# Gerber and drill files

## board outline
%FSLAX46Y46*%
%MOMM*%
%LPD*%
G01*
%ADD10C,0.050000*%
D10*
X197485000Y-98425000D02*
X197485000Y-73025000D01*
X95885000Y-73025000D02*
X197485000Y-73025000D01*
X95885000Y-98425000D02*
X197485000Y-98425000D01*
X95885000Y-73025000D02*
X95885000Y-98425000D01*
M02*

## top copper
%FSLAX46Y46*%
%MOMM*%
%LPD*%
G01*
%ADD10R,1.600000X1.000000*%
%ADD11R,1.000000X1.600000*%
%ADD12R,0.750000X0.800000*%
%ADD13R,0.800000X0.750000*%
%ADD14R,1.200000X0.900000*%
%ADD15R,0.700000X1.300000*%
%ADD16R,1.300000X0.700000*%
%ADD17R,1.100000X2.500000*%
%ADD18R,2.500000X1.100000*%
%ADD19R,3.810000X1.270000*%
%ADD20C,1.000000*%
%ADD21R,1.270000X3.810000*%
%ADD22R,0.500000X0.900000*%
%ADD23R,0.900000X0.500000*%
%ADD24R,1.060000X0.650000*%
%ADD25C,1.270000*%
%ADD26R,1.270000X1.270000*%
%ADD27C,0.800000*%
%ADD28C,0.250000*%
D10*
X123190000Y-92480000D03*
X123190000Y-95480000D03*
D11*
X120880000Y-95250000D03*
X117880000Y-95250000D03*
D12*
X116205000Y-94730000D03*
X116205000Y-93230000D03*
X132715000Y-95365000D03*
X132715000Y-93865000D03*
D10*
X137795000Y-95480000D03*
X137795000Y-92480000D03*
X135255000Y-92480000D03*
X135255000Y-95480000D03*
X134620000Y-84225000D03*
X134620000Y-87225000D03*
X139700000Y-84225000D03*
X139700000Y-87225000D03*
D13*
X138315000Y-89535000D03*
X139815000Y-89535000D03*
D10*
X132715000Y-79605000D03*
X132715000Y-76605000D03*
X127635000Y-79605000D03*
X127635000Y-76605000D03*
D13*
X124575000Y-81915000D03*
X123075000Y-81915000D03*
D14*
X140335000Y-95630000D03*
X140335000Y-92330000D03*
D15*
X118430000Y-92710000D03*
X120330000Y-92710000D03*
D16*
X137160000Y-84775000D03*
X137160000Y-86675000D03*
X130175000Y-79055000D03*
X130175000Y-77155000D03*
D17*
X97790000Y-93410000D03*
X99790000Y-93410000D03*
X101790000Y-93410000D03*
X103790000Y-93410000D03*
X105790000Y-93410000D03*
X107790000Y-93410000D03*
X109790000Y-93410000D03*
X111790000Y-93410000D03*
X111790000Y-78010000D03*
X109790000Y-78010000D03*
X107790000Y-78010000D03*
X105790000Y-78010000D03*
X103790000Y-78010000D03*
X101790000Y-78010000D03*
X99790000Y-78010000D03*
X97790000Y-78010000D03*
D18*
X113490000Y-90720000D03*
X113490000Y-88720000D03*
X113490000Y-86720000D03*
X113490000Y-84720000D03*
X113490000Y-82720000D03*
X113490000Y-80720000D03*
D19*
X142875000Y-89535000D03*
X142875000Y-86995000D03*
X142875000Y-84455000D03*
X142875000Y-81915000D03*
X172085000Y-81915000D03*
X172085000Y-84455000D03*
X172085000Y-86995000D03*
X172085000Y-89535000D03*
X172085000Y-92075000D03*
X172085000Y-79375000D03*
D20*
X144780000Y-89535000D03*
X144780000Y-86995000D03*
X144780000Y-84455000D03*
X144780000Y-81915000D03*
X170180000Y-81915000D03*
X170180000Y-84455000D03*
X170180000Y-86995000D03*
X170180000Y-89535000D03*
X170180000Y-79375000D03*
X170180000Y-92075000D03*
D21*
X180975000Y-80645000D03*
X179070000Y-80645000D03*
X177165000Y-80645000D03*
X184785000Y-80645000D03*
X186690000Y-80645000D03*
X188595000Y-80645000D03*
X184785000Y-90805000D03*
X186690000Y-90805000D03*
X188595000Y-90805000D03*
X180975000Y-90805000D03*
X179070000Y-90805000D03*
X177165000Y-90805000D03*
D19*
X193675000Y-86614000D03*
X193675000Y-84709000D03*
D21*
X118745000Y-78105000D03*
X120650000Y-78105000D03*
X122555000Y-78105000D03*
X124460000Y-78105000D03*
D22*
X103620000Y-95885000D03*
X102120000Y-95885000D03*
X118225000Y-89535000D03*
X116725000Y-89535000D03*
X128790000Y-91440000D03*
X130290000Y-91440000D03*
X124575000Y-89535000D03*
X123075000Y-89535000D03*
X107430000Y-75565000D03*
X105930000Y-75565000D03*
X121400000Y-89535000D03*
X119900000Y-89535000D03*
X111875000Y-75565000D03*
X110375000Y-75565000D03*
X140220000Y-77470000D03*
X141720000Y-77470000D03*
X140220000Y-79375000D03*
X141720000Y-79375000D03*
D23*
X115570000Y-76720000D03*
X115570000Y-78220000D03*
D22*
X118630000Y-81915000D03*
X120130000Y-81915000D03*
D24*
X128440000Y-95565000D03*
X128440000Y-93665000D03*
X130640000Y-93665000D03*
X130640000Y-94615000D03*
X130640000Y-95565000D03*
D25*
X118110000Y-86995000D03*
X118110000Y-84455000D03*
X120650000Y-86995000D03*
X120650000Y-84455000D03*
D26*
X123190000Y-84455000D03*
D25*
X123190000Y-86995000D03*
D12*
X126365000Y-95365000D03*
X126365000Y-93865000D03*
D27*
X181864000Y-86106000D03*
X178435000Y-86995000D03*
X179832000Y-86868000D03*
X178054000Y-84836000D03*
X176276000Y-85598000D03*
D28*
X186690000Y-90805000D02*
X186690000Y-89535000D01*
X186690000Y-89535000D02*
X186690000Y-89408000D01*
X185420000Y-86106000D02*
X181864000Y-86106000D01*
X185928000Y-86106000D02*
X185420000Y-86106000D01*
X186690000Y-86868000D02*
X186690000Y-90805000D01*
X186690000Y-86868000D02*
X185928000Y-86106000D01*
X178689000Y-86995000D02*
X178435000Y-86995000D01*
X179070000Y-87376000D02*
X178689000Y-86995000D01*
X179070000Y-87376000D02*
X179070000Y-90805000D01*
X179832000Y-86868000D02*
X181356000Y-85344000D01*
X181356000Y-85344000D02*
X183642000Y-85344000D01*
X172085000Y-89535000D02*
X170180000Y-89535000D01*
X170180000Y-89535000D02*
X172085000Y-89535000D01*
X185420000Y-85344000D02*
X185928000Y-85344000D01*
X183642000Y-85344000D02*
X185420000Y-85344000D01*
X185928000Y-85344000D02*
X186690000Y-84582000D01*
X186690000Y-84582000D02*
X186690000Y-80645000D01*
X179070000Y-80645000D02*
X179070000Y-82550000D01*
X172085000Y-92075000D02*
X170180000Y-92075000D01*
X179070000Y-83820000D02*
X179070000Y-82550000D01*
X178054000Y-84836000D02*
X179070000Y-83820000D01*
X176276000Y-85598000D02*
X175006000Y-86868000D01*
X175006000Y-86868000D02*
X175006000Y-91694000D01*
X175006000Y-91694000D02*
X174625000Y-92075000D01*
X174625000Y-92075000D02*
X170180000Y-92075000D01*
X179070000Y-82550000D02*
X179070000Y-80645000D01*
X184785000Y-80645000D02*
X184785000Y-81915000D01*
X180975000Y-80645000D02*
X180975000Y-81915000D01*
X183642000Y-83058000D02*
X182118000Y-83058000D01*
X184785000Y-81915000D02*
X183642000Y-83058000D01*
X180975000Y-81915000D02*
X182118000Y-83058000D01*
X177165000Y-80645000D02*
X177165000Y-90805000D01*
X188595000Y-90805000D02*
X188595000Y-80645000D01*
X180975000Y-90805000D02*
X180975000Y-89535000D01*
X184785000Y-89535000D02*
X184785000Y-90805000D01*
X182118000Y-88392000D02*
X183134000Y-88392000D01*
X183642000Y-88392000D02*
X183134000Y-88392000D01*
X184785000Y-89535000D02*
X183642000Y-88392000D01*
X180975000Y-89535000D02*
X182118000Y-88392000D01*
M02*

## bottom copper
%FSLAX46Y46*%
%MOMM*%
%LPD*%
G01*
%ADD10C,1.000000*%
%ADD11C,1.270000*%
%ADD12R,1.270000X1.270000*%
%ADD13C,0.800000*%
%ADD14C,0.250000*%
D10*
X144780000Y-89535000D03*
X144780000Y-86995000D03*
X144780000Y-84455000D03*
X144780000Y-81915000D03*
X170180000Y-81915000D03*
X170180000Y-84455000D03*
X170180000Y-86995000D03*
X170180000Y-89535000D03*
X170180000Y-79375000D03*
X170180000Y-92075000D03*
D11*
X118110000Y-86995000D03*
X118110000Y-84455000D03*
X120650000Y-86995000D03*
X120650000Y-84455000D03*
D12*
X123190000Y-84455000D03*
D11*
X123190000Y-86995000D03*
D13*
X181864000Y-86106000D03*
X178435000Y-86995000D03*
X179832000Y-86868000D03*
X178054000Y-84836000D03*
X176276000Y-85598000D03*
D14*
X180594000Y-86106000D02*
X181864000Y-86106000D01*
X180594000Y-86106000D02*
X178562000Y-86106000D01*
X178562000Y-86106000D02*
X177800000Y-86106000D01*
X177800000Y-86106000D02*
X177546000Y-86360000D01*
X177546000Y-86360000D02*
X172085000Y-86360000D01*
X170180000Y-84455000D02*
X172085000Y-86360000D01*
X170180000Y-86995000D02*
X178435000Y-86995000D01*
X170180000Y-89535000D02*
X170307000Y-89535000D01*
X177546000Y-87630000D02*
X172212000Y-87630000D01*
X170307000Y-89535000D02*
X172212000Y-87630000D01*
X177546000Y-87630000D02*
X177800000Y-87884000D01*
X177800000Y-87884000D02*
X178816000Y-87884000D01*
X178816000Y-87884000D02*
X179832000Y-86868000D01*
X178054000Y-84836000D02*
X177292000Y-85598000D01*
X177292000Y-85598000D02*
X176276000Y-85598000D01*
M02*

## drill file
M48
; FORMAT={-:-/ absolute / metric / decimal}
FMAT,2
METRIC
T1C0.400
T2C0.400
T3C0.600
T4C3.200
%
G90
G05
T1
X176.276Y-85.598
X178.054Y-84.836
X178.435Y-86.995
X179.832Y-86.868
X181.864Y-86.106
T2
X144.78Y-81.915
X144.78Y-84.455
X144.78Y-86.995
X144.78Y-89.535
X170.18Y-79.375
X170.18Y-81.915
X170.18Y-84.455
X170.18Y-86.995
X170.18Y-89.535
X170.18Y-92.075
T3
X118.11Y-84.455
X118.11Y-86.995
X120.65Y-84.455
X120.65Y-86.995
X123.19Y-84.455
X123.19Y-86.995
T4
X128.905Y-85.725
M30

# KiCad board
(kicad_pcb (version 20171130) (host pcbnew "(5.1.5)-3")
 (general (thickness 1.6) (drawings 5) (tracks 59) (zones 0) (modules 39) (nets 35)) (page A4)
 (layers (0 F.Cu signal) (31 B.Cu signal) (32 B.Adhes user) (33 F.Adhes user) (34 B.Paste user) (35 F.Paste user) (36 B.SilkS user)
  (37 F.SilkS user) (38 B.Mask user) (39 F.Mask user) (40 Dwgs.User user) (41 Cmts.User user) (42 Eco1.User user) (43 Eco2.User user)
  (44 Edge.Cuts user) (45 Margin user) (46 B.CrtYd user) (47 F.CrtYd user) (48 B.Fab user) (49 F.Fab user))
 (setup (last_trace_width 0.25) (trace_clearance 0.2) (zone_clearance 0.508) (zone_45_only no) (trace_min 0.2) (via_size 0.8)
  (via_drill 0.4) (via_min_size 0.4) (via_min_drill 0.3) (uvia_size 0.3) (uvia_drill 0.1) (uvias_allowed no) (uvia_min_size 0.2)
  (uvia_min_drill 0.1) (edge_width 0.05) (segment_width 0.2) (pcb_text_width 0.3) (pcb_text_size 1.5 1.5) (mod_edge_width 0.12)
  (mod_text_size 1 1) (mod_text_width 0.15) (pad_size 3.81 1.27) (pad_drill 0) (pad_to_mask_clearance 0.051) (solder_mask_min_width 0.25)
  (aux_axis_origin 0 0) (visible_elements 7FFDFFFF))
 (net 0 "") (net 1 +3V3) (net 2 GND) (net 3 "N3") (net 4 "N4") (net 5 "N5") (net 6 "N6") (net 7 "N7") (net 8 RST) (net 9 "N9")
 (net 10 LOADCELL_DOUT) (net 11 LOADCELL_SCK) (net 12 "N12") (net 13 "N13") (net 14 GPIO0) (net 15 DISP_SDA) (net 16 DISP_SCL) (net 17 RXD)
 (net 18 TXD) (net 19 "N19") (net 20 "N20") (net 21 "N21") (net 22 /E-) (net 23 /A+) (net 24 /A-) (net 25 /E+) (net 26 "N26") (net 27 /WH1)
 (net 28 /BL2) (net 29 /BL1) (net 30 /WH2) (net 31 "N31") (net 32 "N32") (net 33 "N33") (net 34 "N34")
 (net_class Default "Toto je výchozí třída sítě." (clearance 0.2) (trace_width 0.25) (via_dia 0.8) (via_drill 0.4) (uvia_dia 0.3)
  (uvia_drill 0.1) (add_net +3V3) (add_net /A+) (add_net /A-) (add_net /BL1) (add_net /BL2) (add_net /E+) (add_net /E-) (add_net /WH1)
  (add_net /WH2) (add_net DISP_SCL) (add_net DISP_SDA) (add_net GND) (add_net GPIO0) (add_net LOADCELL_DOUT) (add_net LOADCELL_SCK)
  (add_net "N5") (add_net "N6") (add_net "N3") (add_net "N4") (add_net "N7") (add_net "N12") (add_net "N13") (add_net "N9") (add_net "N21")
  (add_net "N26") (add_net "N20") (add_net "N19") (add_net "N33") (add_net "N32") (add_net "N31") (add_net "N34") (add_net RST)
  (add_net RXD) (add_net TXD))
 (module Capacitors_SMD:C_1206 (layer F.Cu) (at 123.19 93.98 270)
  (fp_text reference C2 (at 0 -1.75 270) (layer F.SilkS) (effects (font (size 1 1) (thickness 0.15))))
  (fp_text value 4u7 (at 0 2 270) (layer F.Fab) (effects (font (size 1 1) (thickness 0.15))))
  (pad 1 smd rect (at -1.5 0 270) (size 1 1.6) (layers F.Cu F.Paste F.Mask) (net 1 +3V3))
  (pad 2 smd rect (at 1.5 0 270) (size 1 1.6) (layers F.Cu F.Paste F.Mask) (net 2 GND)))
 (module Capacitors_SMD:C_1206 (layer F.Cu) (at 119.38 95.25)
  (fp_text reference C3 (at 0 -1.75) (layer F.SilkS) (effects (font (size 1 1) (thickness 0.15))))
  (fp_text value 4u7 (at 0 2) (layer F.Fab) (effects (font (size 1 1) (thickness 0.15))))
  (pad 2 smd rect (at 1.5 0) (size 1 1.6) (layers F.Cu F.Paste F.Mask) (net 2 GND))
  (pad 1 smd rect (at -1.5 0) (size 1 1.6) (layers F.Cu F.Paste F.Mask) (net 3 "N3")))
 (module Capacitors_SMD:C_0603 (layer F.Cu) (at 116.205 93.98 90)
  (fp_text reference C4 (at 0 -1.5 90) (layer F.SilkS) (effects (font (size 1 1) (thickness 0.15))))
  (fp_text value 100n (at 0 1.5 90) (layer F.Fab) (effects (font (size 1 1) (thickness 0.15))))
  (pad 1 smd rect (at -0.75 0 90) (size 0.8 0.75) (layers F.Cu F.Paste F.Mask) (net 3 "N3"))
  (pad 2 smd rect (at 0.75 0 90) (size 0.8 0.75) (layers F.Cu F.Paste F.Mask) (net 2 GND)))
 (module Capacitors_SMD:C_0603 (layer F.Cu) (at 132.715 94.615 90)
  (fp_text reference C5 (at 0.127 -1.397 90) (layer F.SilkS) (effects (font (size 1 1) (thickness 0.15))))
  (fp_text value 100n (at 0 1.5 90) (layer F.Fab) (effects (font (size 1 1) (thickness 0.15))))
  (pad 1 smd rect (at -0.75 0 90) (size 0.8 0.75) (layers F.Cu F.Paste F.Mask) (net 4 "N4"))
  (pad 2 smd rect (at 0.75 0 90) (size 0.8 0.75) (layers F.Cu F.Paste F.Mask) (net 2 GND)))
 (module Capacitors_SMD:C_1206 (layer F.Cu) (at 137.795 93.98 90)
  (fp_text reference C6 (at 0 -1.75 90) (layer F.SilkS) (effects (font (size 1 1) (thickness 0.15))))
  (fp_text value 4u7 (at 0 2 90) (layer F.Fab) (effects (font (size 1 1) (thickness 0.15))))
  (pad 1 smd rect (at -1.5 0 90) (size 1 1.6) (layers F.Cu F.Paste F.Mask) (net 4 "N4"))
  (pad 2 smd rect (at 1.5 0 90) (size 1 1.6) (layers F.Cu F.Paste F.Mask) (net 2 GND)))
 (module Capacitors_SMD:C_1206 (layer F.Cu) (at 135.255 93.98 90)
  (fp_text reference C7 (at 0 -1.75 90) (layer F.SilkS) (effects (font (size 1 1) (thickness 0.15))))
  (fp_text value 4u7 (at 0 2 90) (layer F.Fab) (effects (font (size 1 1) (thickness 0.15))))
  (pad 2 smd rect (at 1.5 0 90) (size 1 1.6) (layers F.Cu F.Paste F.Mask) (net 2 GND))
  (pad 1 smd rect (at -1.5 0 90) (size 1 1.6) (layers F.Cu F.Paste F.Mask) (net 4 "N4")))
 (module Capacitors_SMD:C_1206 (layer F.Cu) (at 134.62 85.725 90)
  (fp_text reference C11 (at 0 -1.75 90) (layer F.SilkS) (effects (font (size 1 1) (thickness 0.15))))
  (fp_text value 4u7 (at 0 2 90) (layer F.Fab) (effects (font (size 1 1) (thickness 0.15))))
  (pad 2 smd rect (at 1.5 0 90) (size 1 1.6) (layers F.Cu F.Paste F.Mask) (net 2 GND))
  (pad 1 smd rect (at -1.5 0 90) (size 1 1.6) (layers F.Cu F.Paste F.Mask) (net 1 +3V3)))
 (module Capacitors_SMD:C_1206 (layer F.Cu) (at 139.7 85.725 90)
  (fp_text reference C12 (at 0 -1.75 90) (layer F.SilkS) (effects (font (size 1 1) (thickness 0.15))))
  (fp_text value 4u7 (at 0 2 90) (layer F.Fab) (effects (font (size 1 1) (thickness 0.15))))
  (pad 2 smd rect (at 1.5 0 90) (size 1 1.6) (layers F.Cu F.Paste F.Mask) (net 2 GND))
  (pad 1 smd rect (at -1.5 0 90) (size 1 1.6) (layers F.Cu F.Paste F.Mask) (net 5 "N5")))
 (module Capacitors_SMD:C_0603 (layer F.Cu) (at 139.065 89.535 180)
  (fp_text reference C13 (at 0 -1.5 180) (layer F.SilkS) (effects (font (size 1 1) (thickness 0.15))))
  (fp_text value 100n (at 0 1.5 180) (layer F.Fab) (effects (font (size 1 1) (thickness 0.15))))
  (pad 2 smd rect (at 0.75 0 180) (size 0.8 0.75) (layers F.Cu F.Paste F.Mask) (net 2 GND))
  (pad 1 smd rect (at -0.75 0 180) (size 0.8 0.75) (layers F.Cu F.Paste F.Mask) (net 5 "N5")))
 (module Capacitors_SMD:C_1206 (layer F.Cu) (at 132.715 78.105 90)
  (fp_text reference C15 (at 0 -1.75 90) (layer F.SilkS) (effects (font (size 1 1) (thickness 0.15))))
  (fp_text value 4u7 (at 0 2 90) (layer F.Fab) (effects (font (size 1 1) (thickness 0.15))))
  (pad 1 smd rect (at -1.5 0 90) (size 1 1.6) (layers F.Cu F.Paste F.Mask) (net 1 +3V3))
  (pad 2 smd rect (at 1.5 0 90) (size 1 1.6) (layers F.Cu F.Paste F.Mask) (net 2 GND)))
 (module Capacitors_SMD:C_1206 (layer F.Cu) (at 127.635 78.105 270)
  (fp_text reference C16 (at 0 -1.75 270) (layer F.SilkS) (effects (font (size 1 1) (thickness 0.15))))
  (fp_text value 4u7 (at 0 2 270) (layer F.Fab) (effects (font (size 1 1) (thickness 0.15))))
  (pad 2 smd rect (at 1.5 0 270) (size 1 1.6) (layers F.Cu F.Paste F.Mask) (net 2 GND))
  (pad 1 smd rect (at -1.5 0 270) (size 1 1.6) (layers F.Cu F.Paste F.Mask) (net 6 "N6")))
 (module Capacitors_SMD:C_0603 (layer F.Cu) (at 123.825 81.915)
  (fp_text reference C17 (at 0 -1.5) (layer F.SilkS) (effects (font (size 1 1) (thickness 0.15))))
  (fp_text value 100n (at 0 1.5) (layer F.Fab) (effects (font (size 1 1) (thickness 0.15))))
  (pad 2 smd rect (at 0.75 0) (size 0.8 0.75) (layers F.Cu F.Paste F.Mask) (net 2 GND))
  (pad 1 smd rect (at -0.75 0) (size 0.8 0.75) (layers F.Cu F.Paste F.Mask) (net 6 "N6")))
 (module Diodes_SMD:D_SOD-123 (layer F.Cu) (at 140.335 93.98 270)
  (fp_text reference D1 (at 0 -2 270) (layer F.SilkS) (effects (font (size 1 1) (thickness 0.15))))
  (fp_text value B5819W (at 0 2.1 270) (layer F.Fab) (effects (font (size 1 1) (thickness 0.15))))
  (pad 2 smd rect (at 1.65 0 270) (size 0.9 1.2) (layers F.Cu F.Paste F.Mask) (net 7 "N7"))
  (pad 1 smd rect (at -1.65 0 270) (size 0.9 1.2) (layers F.Cu F.Paste F.Mask) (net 4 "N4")))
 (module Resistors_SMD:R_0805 (layer F.Cu) (at 119.38 92.71)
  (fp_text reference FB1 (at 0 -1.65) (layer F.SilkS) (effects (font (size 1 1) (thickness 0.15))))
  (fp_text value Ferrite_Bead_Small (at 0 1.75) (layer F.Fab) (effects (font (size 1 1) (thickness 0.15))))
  (pad 1 smd rect (at -0.95 0) (size 0.7 1.3) (layers F.Cu F.Paste F.Mask) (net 3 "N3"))
  (pad 2 smd rect (at 0.95 0) (size 0.7 1.3) (layers F.Cu F.Paste F.Mask) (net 1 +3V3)))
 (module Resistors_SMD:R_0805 (layer F.Cu) (at 137.16 85.725 90)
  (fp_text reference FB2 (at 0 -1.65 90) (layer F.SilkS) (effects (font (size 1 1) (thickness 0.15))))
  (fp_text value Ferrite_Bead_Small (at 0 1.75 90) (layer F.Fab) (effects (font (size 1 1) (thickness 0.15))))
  (pad 2 smd rect (at 0.95 0 90) (size 0.7 1.3) (layers F.Cu F.Paste F.Mask) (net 1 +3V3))
  (pad 1 smd rect (at -0.95 0 90) (size 0.7 1.3) (layers F.Cu F.Paste F.Mask) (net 5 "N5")))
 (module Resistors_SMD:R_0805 (layer F.Cu) (at 130.175 78.105 270)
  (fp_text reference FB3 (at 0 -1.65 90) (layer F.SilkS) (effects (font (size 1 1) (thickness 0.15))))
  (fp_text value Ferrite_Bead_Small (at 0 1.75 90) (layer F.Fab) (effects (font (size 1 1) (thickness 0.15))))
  (pad 2 smd rect (at 0.95 0 270) (size 0.7 1.3) (layers F.Cu F.Paste F.Mask) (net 1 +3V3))
  (pad 1 smd rect (at -0.95 0 270) (size 0.7 1.3) (layers F.Cu F.Paste F.Mask) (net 6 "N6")))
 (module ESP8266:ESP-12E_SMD (layer F.Cu) (at 97.79 92.71 90)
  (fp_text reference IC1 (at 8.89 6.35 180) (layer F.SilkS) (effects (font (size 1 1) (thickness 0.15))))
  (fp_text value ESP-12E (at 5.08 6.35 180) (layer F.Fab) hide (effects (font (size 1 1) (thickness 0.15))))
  (pad 1 smd rect (at 0 0 90) (size 2.5 1.1) (drill (offset -0.7 0)) (layers F.Cu F.Paste F.Mask) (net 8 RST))
  (pad 2 smd rect (at 0 2 90) (size 2.5 1.1) (drill (offset -0.7 0)) (layers F.Cu F.Paste F.Mask))
  (pad 3 smd rect (at 0 4 90) (size 2.5 1.1) (drill (offset -0.7 0)) (layers F.Cu F.Paste F.Mask) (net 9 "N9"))
  (pad 4 smd rect (at 0 6 90) (size 2.5 1.1) (drill (offset -0.7 0)) (layers F.Cu F.Paste F.Mask))
  (pad 5 smd rect (at 0 8 90) (size 2.5 1.1) (drill (offset -0.7 0)) (layers F.Cu F.Paste F.Mask) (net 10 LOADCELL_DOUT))
  (pad 6 smd rect (at 0 10 90) (size 2.5 1.1) (drill (offset -0.7 0)) (layers F.Cu F.Paste F.Mask) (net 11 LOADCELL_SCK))
  (pad 7 smd rect (at 0 12 90) (size 2.5 1.1) (drill (offset -0.7 0)) (layers F.Cu F.Paste F.Mask))
  (pad 8 smd rect (at 0 14 90) (size 2.5 1.1) (drill (offset -0.7 0)) (layers F.Cu F.Paste F.Mask) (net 3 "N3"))
  (pad 9 smd rect (at 14 14 90) (size 2.5 1.1) (drill (offset 0.7 0)) (layers F.Cu F.Paste F.Mask) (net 2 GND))
  (pad 10 smd rect (at 14 12 90) (size 2.5 1.1) (drill (offset 0.7 0)) (layers F.Cu F.Paste F.Mask) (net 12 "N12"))
  (pad 11 smd rect (at 14 10 90) (size 2.5 1.1) (drill (offset 0.7 0)) (layers F.Cu F.Paste F.Mask) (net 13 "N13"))
  (pad 12 smd rect (at 14 8 90) (size 2.5 1.1) (drill (offset 0.7 0)) (layers F.Cu F.Paste F.Mask) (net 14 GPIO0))
  (pad 13 smd rect (at 14 6 90) (size 2.5 1.1) (drill (offset 0.7 0)) (layers F.Cu F.Paste F.Mask) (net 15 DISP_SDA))
  (pad 14 smd rect (at 14 4 90) (size 2.5 1.1) (drill (offset 0.7 0)) (layers F.Cu F.Paste F.Mask) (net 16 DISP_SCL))
  (pad 15 smd rect (at 14 2 90) (size 2.5 1.1) (drill (offset 0.7 0)) (layers F.Cu F.Paste F.Mask) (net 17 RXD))
  (pad 16 smd rect (at 14 0 90) (size 2.5 1.1) (drill (offset 0.7 0)) (layers F.Cu F.Paste F.Mask) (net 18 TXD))
  (pad 17 smd rect (at 1.99 15 180) (size 2.5 1.1) (drill (offset -0.7 0)) (layers F.Cu F.Paste F.Mask))
  (pad 18 smd rect (at 3.99 15 180) (size 2.5 1.1) (drill (offset -0.7 0)) (layers F.Cu F.Paste F.Mask))
  (pad 19 smd rect (at 5.99 15 180) (size 2.5 1.1) (drill (offset -0.7 0)) (layers F.Cu F.Paste F.Mask))
  (pad 20 smd rect (at 7.99 15 180) (size 2.5 1.1) (drill (offset -0.7 0)) (layers F.Cu F.Paste F.Mask))
  (pad 21 smd rect (at 9.99 15 180) (size 2.5 1.1) (drill (offset -0.7 0)) (layers F.Cu F.Paste F.Mask))
  (pad 22 smd rect (at 11.99 15 180) (size 2.5 1.1) (drill (offset -0.7 0)) (layers F.Cu F.Paste F.Mask)))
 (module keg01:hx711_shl (layer F.Cu) (at 157.48 85.725)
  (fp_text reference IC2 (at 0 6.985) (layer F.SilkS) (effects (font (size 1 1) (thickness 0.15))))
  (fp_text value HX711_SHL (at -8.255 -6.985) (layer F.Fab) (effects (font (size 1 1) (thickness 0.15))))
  (pad 5 smd rect (at -14.605 3.81) (size 3.81 1.27) (layers F.Cu F.Paste F.Mask) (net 5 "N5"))
  (pad 4 smd rect (at -14.605 1.27) (size 3.81 1.27) (layers F.Cu F.Paste F.Mask) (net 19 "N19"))
  (pad 3 smd rect (at -14.605 -1.27) (size 3.81 1.27) (layers F.Cu F.Paste F.Mask) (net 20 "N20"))
  (pad 2 smd rect (at -14.605 -3.81) (size 3.81 1.27) (layers F.Cu F.Paste F.Mask) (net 2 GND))
  (pad 11 smd rect (at 14.605 -3.81) (size 3.81 1.27) (layers F.Cu F.Paste F.Mask) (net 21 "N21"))
  (pad 10 smd rect (at 14.605 -1.27) (size 3.81 1.27) (layers F.Cu F.Paste F.Mask) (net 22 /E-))
  (pad 9 smd rect (at 14.605 1.27) (size 3.81 1.27) (layers F.Cu F.Paste F.Mask) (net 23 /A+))
  (pad 8 smd rect (at 14.605 3.81) (size 3.81 1.27) (layers F.Cu F.Paste F.Mask) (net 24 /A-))
  (pad 7 smd rect (at 14.605 6.35) (size 3.81 1.27) (layers F.Cu F.Paste F.Mask) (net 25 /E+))
  (pad 12 smd rect (at 14.605 -6.35) (size 3.81 1.27) (layers F.Cu F.Paste F.Mask) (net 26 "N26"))
  (pad 5 thru_hole circle (at -12.7 3.81) (size 1 1) (drill 0.4) (layers *.Cu *.Mask) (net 5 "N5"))
  (pad 4 thru_hole circle (at -12.7 1.27) (size 1 1) (drill 0.4) (layers *.Cu *.Mask) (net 19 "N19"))
  (pad 3 thru_hole circle (at -12.7 -1.27) (size 1 1) (drill 0.4) (layers *.Cu *.Mask) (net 20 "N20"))
  (pad 2 thru_hole circle (at -12.7 -3.81) (size 1 1) (drill 0.4) (layers *.Cu *.Mask) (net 2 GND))
  (pad 11 thru_hole circle (at 12.7 -3.81) (size 1 1) (drill 0.4) (layers *.Cu *.Mask) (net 21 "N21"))
  (pad 10 thru_hole circle (at 12.7 -1.27) (size 1 1) (drill 0.4) (layers *.Cu *.Mask) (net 22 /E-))
  (pad 9 thru_hole circle (at 12.7 1.27) (size 1 1) (drill 0.4) (layers *.Cu *.Mask) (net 23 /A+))
  (pad 8 thru_hole circle (at 12.7 3.81) (size 1 1) (drill 0.4) (layers *.Cu *.Mask) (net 24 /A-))
  (pad 12 thru_hole circle (at 12.7 -6.35) (size 1 1) (drill 0.4) (layers *.Cu *.Mask) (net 26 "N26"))
  (pad 7 thru_hole circle (at 12.7 6.35) (size 1 1) (drill 0.4) (layers *.Cu *.Mask) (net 25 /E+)))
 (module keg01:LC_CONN (layer F.Cu) (at 179.07 80.645 90)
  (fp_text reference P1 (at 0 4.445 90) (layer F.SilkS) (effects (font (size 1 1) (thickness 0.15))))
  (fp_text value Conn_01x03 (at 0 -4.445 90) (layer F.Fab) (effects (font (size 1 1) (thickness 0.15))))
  (pad 3 smd rect (at 0 1.905 90) (size 3.81 1.27) (layers F.Cu F.Paste F.Mask) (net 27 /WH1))
  (pad 2 smd rect (at 0 0 90) (size 3.81 1.27) (layers F.Cu F.Paste F.Mask) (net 25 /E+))
  (pad 1 smd rect (at 0 -1.905 90) (size 3.81 1.27) (layers F.Cu F.Paste F.Mask) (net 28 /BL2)))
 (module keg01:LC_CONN (layer F.Cu) (at 186.69 80.645 90)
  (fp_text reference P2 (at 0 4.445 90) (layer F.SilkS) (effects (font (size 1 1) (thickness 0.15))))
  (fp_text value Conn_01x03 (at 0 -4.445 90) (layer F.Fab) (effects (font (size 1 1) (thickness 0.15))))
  (pad 1 smd rect (at 0 -1.905 90) (size 3.81 1.27) (layers F.Cu F.Paste F.Mask) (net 27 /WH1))
  (pad 2 smd rect (at 0 0 90) (size 3.81 1.27) (layers F.Cu F.Paste F.Mask) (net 24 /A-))
  (pad 3 smd rect (at 0 1.905 90) (size 3.81 1.27) (layers F.Cu F.Paste F.Mask) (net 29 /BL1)))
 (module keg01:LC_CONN (layer F.Cu) (at 186.69 90.805 270)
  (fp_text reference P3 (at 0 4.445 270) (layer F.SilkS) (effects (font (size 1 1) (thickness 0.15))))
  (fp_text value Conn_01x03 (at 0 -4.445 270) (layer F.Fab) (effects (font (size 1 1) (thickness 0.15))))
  (pad 3 smd rect (at 0 1.905 270) (size 3.81 1.27) (layers F.Cu F.Paste F.Mask) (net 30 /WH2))
  (pad 2 smd rect (at 0 0 270) (size 3.81 1.27) (layers F.Cu F.Paste F.Mask) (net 22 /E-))
  (pad 1 smd rect (at 0 -1.905 270) (size 3.81 1.27) (layers F.Cu F.Paste F.Mask) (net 29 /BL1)))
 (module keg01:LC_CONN (layer F.Cu) (at 179.07 90.805 270)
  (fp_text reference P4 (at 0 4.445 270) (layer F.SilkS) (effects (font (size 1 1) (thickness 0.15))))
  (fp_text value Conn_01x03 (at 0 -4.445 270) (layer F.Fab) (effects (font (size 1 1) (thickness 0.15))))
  (pad 1 smd rect (at 0 -1.905 270) (size 3.81 1.27) (layers F.Cu F.Paste F.Mask) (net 30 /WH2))
  (pad 2 smd rect (at 0 0 270) (size 3.81 1.27) (layers F.Cu F.Paste F.Mask) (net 23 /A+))
  (pad 3 smd rect (at 0 1.905 270) (size 3.81 1.27) (layers F.Cu F.Paste F.Mask) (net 28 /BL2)))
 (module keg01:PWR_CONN (layer F.Cu) (at 193.675 85.979 180)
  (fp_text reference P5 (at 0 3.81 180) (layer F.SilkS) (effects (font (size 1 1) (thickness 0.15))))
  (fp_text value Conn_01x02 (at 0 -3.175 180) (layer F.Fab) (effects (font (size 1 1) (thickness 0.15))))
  (pad 2 smd rect (at 0 -0.635 180) (size 3.81 1.27) (layers F.Cu F.Paste F.Mask) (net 7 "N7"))
  (pad 1 smd rect (at 0 1.27 180) (size 3.81 1.27) (layers F.Cu F.Paste F.Mask) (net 2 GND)))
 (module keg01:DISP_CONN (layer F.Cu) (at 121.285 78.105 90)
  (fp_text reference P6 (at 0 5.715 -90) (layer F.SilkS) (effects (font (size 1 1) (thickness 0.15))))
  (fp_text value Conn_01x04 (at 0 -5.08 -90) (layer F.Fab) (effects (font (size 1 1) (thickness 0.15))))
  (pad 4 smd rect (at 0 -2.54 90) (size 3.81 1.27) (layers F.Cu F.Paste F.Mask) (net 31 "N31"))
  (pad 3 smd rect (at 0 -0.635 90) (size 3.81 1.27) (layers F.Cu F.Paste F.Mask) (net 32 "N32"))
  (pad 2 smd rect (at 0 1.27 90) (size 3.81 1.27) (layers F.Cu F.Paste F.Mask) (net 6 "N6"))
  (pad 1 smd rect (at 0 3.175 90) (size 3.81 1.27) (layers F.Cu F.Paste F.Mask) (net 2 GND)))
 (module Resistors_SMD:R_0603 (layer F.Cu) (at 102.87 95.885 180)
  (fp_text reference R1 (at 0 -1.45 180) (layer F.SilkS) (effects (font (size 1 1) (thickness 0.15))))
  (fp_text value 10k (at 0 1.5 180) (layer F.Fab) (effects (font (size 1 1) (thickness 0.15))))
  (pad 1 smd rect (at -0.75 0 180) (size 0.5 0.9) (layers F.Cu F.Paste F.Mask) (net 1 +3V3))
  (pad 2 smd rect (at 0.75 0 180) (size 0.5 0.9) (layers F.Cu F.Paste F.Mask) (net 9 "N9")))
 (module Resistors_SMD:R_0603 (layer F.Cu) (at 117.475 89.535 180)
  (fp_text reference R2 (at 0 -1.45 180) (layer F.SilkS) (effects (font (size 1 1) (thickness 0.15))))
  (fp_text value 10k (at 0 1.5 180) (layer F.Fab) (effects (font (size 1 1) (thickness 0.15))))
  (pad 1 smd rect (at -0.75 0 180) (size 0.5 0.9) (layers F.Cu F.Paste F.Mask) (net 1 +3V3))
  (pad 2 smd rect (at 0.75 0 180) (size 0.5 0.9) (layers F.Cu F.Paste F.Mask) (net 8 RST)))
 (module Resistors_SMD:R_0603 (layer F.Cu) (at 129.54 91.44 180)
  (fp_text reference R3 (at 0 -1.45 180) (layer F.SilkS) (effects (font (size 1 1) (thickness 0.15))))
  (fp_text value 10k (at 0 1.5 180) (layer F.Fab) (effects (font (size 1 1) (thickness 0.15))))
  (pad 2 smd rect (at 0.75 0 180) (size 0.5 0.9) (layers F.Cu F.Paste F.Mask) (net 4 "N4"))
  (pad 1 smd rect (at -0.75 0 180) (size 0.5 0.9) (layers F.Cu F.Paste F.Mask) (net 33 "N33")))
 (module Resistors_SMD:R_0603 (layer F.Cu) (at 123.825 89.535 180)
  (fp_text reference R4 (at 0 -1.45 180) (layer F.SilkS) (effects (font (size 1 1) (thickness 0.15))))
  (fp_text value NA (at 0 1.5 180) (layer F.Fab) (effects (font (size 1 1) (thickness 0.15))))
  (pad 1 smd rect (at -0.75 0 180) (size 0.5 0.9) (layers F.Cu F.Paste F.Mask) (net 1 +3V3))
  (pad 2 smd rect (at 0.75 0 180) (size 0.5 0.9) (layers F.Cu F.Paste F.Mask) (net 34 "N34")))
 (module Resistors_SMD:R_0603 (layer F.Cu) (at 106.68 75.565)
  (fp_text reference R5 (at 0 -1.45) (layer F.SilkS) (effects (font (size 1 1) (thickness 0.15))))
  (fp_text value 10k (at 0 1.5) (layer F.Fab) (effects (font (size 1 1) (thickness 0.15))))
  (pad 2 smd rect (at 0.75 0) (size 0.5 0.9) (layers F.Cu F.Paste F.Mask) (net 13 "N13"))
  (pad 1 smd rect (at -0.75 0) (size 0.5 0.9) (layers F.Cu F.Paste F.Mask) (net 1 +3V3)))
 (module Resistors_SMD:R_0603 (layer F.Cu) (at 120.65 89.535 180)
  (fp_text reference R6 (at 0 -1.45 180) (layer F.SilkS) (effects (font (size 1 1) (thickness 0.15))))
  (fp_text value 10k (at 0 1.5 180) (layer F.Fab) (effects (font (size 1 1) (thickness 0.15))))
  (pad 1 smd rect (at -0.75 0 180) (size 0.5 0.9) (layers F.Cu F.Paste F.Mask) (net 1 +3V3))
  (pad 2 smd rect (at 0.75 0 180) (size 0.5 0.9) (layers F.Cu F.Paste F.Mask) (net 14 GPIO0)))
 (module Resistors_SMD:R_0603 (layer F.Cu) (at 111.125 75.565)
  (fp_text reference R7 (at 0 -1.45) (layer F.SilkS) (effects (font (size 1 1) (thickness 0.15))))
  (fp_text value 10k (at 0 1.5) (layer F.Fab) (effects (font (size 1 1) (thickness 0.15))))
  (pad 2 smd rect (at 0.75 0) (size 0.5 0.9) (layers F.Cu F.Paste F.Mask) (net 2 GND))
  (pad 1 smd rect (at -0.75 0) (size 0.5 0.9) (layers F.Cu F.Paste F.Mask) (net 12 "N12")))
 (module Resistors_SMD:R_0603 (layer F.Cu) (at 140.97 77.47 180)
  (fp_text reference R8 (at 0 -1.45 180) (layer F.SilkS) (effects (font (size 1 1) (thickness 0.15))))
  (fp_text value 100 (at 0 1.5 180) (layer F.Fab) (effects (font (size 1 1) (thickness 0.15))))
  (pad 2 smd rect (at 0.75 0 180) (size 0.5 0.9) (layers F.Cu F.Paste F.Mask) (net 10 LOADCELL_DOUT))
  (pad 1 smd rect (at -0.75 0 180) (size 0.5 0.9) (layers F.Cu F.Paste F.Mask) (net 19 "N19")))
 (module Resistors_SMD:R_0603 (layer F.Cu) (at 140.97 79.375 180)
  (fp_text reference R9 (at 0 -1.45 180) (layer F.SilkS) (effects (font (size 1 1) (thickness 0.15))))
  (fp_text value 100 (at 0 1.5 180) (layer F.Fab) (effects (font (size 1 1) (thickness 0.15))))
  (pad 2 smd rect (at 0.75 0 180) (size 0.5 0.9) (layers F.Cu F.Paste F.Mask) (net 11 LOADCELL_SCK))
  (pad 1 smd rect (at -0.75 0 180) (size 0.5 0.9) (layers F.Cu F.Paste F.Mask) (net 20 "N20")))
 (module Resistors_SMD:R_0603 (layer F.Cu) (at 115.57 77.47 270)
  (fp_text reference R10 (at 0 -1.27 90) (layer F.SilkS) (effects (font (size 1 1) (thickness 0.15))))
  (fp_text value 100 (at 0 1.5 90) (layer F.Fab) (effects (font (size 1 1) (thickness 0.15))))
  (pad 1 smd rect (at -0.75 0 270) (size 0.5 0.9) (layers F.Cu F.Paste F.Mask) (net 31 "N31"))
  (pad 2 smd rect (at 0.75 0 270) (size 0.5 0.9) (layers F.Cu F.Paste F.Mask) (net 15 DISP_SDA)))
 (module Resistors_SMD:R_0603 (layer F.Cu) (at 119.38 81.915 180)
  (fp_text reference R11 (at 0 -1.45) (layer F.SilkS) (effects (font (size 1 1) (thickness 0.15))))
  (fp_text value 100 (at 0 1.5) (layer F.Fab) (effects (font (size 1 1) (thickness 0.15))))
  (pad 2 smd rect (at 0.75 0 180) (size 0.5 0.9) (layers F.Cu F.Paste F.Mask) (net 16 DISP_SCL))
  (pad 1 smd rect (at -0.75 0 180) (size 0.5 0.9) (layers F.Cu F.Paste F.Mask) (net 32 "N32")))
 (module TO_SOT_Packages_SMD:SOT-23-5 (layer F.Cu) (at 129.54 94.615 180)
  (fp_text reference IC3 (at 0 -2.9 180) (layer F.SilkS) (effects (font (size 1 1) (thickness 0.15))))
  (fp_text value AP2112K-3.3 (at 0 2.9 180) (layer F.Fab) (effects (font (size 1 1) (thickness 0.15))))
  (pad 5 smd rect (at 1.1 -0.95 180) (size 1.06 0.65) (layers F.Cu F.Paste F.Mask) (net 1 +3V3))
  (pad 4 smd rect (at 1.1 0.95 180) (size 1.06 0.65) (layers F.Cu F.Paste F.Mask))
  (pad 3 smd rect (at -1.1 0.95 180) (size 1.06 0.65) (layers F.Cu F.Paste F.Mask) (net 33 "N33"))
  (pad 2 smd rect (at -1.1 0 180) (size 1.06 0.65) (layers F.Cu F.Paste F.Mask) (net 2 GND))
  (pad 1 smd rect (at -1.1 -0.95 180) (size 1.06 0.65) (layers F.Cu F.Paste F.Mask) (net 4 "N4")))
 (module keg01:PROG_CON (layer F.Cu) (at 120.65 85.725 270)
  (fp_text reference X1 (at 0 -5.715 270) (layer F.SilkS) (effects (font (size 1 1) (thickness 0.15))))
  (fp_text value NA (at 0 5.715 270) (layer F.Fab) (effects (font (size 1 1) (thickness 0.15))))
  (pad 6 thru_hole circle (at 1.27 2.54 270) (size 1.27 1.27) (drill 0.6) (layers *.Cu *.Mask) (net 18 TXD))
  (pad 5 thru_hole circle (at -1.27 2.54 270) (size 1.27 1.27) (drill 0.6) (layers *.Cu *.Mask) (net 17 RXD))
  (pad 4 thru_hole circle (at 1.27 0 270) (size 1.27 1.27) (drill 0.6) (layers *.Cu *.Mask) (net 14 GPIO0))
  (pad 3 thru_hole circle (at -1.27 0 270) (size 1.27 1.27) (drill 0.6) (layers *.Cu *.Mask) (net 8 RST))
  (pad 1 thru_hole rect (at -1.27 -2.54 270) (size 1.27 1.27) (drill 0.6) (layers *.Cu *.Mask) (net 2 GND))
  (pad 2 thru_hole circle (at 1.27 -2.54 270) (size 1.27 1.27) (drill 0.6) (layers *.Cu *.Mask) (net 34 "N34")))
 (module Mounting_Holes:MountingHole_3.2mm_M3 (layer F.Cu) (at 128.905 85.725)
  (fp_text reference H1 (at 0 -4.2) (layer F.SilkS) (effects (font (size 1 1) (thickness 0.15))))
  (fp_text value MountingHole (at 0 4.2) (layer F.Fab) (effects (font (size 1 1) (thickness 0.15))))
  (pad 1 np_thru_hole circle (at 0 0) (size 3.2 3.2) (drill 3.2) (layers *.Cu *.Mask)))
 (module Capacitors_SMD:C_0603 (layer F.Cu) (at 126.365 94.615 90)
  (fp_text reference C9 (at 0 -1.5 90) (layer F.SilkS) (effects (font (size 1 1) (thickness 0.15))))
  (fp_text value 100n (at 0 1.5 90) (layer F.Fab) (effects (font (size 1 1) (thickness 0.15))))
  (pad 1 smd rect (at -0.75 0 90) (size 0.8 0.75) (layers F.Cu F.Paste F.Mask) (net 1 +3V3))
  (pad 2 smd rect (at 0.75 0 90) (size 0.8 0.75) (layers F.Cu F.Paste F.Mask) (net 2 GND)))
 (gr_line (start 197.485 98.425) (end 197.485 73.025) (angle 90) (layer Edge.Cuts) (width 0.05))
 (gr_line (start 95.885 73.025) (end 197.485 73.025) (angle 90) (layer Edge.Cuts) (width 0.05))
 (gr_line (start 95.885 98.425) (end 197.485 98.425) (angle 90) (layer Edge.Cuts) (width 0.05))
 (gr_line (start 95.885 73.025) (end 95.885 98.425) (angle 90) (layer Edge.Cuts) (width 0.05))
 (segment (start 186.69 90.805) (end 186.69 89.535) (width 0.25) (layer F.Cu) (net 22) (status 400030))
 (segment (start 180.594 86.106) (end 181.864 86.106) (width 0.25) (layer B.Cu) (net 22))
 (via (at 181.864 86.106) (size 0.8) (drill 0.4) (layers F.Cu B.Cu) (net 22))
 (segment (start 180.594 86.106) (end 178.562 86.106) (width 0.25) (layer B.Cu) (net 22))
 (segment (start 178.562 86.106) (end 177.8 86.106) (width 0.25) (layer B.Cu) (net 22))
 (segment (start 177.8 86.106) (end 177.546 86.36) (width 0.25) (layer B.Cu) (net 22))
 (segment (start 177.546 86.36) (end 172.085 86.36) (width 0.25) (layer B.Cu) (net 22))
 (segment (start 170.18 84.455) (end 172.085 86.36) (width 0.25) (layer B.Cu) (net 22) (status 400000))
 (segment (start 186.69 89.535) (end 186.69 89.408) (width 0.25) (layer F.Cu) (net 22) (status 30))
 (segment (start 185.42 86.106) (end 181.864 86.106) (width 0.25) (layer F.Cu) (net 22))
 (segment (start 185.928 86.106) (end 185.42 86.106) (width 0.25) (layer F.Cu) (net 22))
 (segment (start 186.69 86.868) (end 186.69 90.805) (width 0.25) (layer F.Cu) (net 22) (status 800020))
 (segment (start 186.69 86.868) (end 185.928 86.106) (width 0.25) (layer F.Cu) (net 22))
 (segment (start 170.18 86.995) (end 178.435 86.995) (width 0.25) (layer B.Cu) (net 23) (status 400000))
 (segment (start 178.689 86.995) (end 178.435 86.995) (width 0.25) (layer F.Cu) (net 23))
 (segment (start 179.07 87.376) (end 178.689 86.995) (width 0.25) (layer F.Cu) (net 23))
 (segment (start 179.07 87.376) (end 179.07 90.805) (width 0.25) (layer F.Cu) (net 23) (status 800020))
 (via (at 178.435 86.995) (size 0.8) (drill 0.4) (layers F.Cu B.Cu) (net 23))
 (segment (start 170.18 89.535) (end 170.307 89.535) (width 0.25) (layer B.Cu) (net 24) (status C00000))
 (segment (start 177.546 87.63) (end 172.212 87.63) (width 0.25) (layer B.Cu) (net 24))
 (segment (start 170.307 89.535) (end 172.212 87.63) (width 0.25) (layer B.Cu) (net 24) (status 400000))
 (segment (start 177.546 87.63) (end 177.8 87.884) (width 0.25) (layer B.Cu) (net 24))
 (segment (start 177.8 87.884) (end 178.816 87.884) (width 0.25) (layer B.Cu) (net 24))
 (segment (start 178.816 87.884) (end 179.832 86.868) (width 0.25) (layer B.Cu) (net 24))
 (via (at 179.832 86.868) (size 0.8) (drill 0.4) (layers F.Cu B.Cu) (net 24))
 (segment (start 179.832 86.868) (end 181.356 85.344) (width 0.25) (layer F.Cu) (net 24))
 (segment (start 181.356 85.344) (end 183.642 85.344) (width 0.25) (layer F.Cu) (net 24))
 (segment (start 172.085 89.535) (end 170.18 89.535) (width 0.25) (layer F.Cu) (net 24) (status C00000))
 (segment (start 170.18 89.535) (end 172.085 89.535) (width 0.25) (layer F.Cu) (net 24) (status C00000))
 (segment (start 185.42 85.344) (end 185.928 85.344) (width 0.25) (layer F.Cu) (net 24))
 (segment (start 183.642 85.344) (end 185.42 85.344) (width 0.25) (layer F.Cu) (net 24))
 (segment (start 185.928 85.344) (end 186.69 84.582) (width 0.25) (layer F.Cu) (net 24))
 (segment (start 186.69 84.582) (end 186.69 80.645) (width 0.25) (layer F.Cu) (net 24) (status 800020))
 (segment (start 179.07 80.645) (end 179.07 82.55) (width 0.25) (layer F.Cu) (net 25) (status 400030))
 (segment (start 172.085 92.075) (end 170.18 92.075) (width 0.25) (layer F.Cu) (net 25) (status C00000))
 (segment (start 179.07 83.82) (end 179.07 82.55) (width 0.25) (layer F.Cu) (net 25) (status 800000))
 (segment (start 178.054 84.836) (end 179.07 83.82) (width 0.25) (layer F.Cu) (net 25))
 (via (at 178.054 84.836) (size 0.8) (drill 0.4) (layers F.Cu B.Cu) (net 25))
 (segment (start 178.054 84.836) (end 177.292 85.598) (width 0.25) (layer B.Cu) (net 25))
 (segment (start 177.292 85.598) (end 176.276 85.598) (width 0.25) (layer B.Cu) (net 25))
 (via (at 176.276 85.598) (size 0.8) (drill 0.4) (layers F.Cu B.Cu) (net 25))
 (segment (start 176.276 85.598) (end 175.006 86.868) (width 0.25) (layer F.Cu) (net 25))
 (segment (start 175.006 86.868) (end 175.006 91.694) (width 0.25) (layer F.Cu) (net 25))
 (segment (start 175.006 91.694) (end 174.625 92.075) (width 0.25) (layer F.Cu) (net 25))
 (segment (start 174.625 92.075) (end 170.18 92.075) (width 0.25) (layer F.Cu) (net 25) (status 800000))
 (segment (start 179.07 82.55) (end 179.07 80.645) (width 0.25) (layer F.Cu) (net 25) (status C00000))
 (segment (start 184.785 80.645) (end 184.785 81.915) (width 0.25) (layer F.Cu) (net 27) (status C00030))
 (segment (start 180.975 80.645) (end 180.975 81.915) (width 0.25) (layer F.Cu) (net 27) (status C00030))
 (segment (start 183.642 83.058) (end 182.118 83.058) (width 0.25) (layer F.Cu) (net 27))
 (segment (start 184.785 81.915) (end 183.642 83.058) (width 0.25) (layer F.Cu) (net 27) (status 10))
 (segment (start 180.975 81.915) (end 182.118 83.058) (width 0.25) (layer F.Cu) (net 27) (status 10))
 (segment (start 177.165 80.645) (end 177.165 90.805) (width 0.25) (layer F.Cu) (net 28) (status C00010))
 (segment (start 188.595 90.805) (end 188.595 80.645) (width 0.25) (layer F.Cu) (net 29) (status C00020))
 (segment (start 180.975 90.805) (end 180.975 89.535) (width 0.25) (layer F.Cu) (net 30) (status C00030))
 (segment (start 184.785 89.535) (end 184.785 90.805) (width 0.25) (layer F.Cu) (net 30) (status C00030))
 (segment (start 182.118 88.392) (end 183.134 88.392) (width 0.25) (layer F.Cu) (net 30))
 (segment (start 183.642 88.392) (end 183.134 88.392) (width 0.25) (layer F.Cu) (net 30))
 (segment (start 184.785 89.535) (end 183.642 88.392) (width 0.25) (layer F.Cu) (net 30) (status 10))
 (segment (start 180.975 89.535) (end 182.118 88.392) (width 0.25) (layer F.Cu) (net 30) (status 10)))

